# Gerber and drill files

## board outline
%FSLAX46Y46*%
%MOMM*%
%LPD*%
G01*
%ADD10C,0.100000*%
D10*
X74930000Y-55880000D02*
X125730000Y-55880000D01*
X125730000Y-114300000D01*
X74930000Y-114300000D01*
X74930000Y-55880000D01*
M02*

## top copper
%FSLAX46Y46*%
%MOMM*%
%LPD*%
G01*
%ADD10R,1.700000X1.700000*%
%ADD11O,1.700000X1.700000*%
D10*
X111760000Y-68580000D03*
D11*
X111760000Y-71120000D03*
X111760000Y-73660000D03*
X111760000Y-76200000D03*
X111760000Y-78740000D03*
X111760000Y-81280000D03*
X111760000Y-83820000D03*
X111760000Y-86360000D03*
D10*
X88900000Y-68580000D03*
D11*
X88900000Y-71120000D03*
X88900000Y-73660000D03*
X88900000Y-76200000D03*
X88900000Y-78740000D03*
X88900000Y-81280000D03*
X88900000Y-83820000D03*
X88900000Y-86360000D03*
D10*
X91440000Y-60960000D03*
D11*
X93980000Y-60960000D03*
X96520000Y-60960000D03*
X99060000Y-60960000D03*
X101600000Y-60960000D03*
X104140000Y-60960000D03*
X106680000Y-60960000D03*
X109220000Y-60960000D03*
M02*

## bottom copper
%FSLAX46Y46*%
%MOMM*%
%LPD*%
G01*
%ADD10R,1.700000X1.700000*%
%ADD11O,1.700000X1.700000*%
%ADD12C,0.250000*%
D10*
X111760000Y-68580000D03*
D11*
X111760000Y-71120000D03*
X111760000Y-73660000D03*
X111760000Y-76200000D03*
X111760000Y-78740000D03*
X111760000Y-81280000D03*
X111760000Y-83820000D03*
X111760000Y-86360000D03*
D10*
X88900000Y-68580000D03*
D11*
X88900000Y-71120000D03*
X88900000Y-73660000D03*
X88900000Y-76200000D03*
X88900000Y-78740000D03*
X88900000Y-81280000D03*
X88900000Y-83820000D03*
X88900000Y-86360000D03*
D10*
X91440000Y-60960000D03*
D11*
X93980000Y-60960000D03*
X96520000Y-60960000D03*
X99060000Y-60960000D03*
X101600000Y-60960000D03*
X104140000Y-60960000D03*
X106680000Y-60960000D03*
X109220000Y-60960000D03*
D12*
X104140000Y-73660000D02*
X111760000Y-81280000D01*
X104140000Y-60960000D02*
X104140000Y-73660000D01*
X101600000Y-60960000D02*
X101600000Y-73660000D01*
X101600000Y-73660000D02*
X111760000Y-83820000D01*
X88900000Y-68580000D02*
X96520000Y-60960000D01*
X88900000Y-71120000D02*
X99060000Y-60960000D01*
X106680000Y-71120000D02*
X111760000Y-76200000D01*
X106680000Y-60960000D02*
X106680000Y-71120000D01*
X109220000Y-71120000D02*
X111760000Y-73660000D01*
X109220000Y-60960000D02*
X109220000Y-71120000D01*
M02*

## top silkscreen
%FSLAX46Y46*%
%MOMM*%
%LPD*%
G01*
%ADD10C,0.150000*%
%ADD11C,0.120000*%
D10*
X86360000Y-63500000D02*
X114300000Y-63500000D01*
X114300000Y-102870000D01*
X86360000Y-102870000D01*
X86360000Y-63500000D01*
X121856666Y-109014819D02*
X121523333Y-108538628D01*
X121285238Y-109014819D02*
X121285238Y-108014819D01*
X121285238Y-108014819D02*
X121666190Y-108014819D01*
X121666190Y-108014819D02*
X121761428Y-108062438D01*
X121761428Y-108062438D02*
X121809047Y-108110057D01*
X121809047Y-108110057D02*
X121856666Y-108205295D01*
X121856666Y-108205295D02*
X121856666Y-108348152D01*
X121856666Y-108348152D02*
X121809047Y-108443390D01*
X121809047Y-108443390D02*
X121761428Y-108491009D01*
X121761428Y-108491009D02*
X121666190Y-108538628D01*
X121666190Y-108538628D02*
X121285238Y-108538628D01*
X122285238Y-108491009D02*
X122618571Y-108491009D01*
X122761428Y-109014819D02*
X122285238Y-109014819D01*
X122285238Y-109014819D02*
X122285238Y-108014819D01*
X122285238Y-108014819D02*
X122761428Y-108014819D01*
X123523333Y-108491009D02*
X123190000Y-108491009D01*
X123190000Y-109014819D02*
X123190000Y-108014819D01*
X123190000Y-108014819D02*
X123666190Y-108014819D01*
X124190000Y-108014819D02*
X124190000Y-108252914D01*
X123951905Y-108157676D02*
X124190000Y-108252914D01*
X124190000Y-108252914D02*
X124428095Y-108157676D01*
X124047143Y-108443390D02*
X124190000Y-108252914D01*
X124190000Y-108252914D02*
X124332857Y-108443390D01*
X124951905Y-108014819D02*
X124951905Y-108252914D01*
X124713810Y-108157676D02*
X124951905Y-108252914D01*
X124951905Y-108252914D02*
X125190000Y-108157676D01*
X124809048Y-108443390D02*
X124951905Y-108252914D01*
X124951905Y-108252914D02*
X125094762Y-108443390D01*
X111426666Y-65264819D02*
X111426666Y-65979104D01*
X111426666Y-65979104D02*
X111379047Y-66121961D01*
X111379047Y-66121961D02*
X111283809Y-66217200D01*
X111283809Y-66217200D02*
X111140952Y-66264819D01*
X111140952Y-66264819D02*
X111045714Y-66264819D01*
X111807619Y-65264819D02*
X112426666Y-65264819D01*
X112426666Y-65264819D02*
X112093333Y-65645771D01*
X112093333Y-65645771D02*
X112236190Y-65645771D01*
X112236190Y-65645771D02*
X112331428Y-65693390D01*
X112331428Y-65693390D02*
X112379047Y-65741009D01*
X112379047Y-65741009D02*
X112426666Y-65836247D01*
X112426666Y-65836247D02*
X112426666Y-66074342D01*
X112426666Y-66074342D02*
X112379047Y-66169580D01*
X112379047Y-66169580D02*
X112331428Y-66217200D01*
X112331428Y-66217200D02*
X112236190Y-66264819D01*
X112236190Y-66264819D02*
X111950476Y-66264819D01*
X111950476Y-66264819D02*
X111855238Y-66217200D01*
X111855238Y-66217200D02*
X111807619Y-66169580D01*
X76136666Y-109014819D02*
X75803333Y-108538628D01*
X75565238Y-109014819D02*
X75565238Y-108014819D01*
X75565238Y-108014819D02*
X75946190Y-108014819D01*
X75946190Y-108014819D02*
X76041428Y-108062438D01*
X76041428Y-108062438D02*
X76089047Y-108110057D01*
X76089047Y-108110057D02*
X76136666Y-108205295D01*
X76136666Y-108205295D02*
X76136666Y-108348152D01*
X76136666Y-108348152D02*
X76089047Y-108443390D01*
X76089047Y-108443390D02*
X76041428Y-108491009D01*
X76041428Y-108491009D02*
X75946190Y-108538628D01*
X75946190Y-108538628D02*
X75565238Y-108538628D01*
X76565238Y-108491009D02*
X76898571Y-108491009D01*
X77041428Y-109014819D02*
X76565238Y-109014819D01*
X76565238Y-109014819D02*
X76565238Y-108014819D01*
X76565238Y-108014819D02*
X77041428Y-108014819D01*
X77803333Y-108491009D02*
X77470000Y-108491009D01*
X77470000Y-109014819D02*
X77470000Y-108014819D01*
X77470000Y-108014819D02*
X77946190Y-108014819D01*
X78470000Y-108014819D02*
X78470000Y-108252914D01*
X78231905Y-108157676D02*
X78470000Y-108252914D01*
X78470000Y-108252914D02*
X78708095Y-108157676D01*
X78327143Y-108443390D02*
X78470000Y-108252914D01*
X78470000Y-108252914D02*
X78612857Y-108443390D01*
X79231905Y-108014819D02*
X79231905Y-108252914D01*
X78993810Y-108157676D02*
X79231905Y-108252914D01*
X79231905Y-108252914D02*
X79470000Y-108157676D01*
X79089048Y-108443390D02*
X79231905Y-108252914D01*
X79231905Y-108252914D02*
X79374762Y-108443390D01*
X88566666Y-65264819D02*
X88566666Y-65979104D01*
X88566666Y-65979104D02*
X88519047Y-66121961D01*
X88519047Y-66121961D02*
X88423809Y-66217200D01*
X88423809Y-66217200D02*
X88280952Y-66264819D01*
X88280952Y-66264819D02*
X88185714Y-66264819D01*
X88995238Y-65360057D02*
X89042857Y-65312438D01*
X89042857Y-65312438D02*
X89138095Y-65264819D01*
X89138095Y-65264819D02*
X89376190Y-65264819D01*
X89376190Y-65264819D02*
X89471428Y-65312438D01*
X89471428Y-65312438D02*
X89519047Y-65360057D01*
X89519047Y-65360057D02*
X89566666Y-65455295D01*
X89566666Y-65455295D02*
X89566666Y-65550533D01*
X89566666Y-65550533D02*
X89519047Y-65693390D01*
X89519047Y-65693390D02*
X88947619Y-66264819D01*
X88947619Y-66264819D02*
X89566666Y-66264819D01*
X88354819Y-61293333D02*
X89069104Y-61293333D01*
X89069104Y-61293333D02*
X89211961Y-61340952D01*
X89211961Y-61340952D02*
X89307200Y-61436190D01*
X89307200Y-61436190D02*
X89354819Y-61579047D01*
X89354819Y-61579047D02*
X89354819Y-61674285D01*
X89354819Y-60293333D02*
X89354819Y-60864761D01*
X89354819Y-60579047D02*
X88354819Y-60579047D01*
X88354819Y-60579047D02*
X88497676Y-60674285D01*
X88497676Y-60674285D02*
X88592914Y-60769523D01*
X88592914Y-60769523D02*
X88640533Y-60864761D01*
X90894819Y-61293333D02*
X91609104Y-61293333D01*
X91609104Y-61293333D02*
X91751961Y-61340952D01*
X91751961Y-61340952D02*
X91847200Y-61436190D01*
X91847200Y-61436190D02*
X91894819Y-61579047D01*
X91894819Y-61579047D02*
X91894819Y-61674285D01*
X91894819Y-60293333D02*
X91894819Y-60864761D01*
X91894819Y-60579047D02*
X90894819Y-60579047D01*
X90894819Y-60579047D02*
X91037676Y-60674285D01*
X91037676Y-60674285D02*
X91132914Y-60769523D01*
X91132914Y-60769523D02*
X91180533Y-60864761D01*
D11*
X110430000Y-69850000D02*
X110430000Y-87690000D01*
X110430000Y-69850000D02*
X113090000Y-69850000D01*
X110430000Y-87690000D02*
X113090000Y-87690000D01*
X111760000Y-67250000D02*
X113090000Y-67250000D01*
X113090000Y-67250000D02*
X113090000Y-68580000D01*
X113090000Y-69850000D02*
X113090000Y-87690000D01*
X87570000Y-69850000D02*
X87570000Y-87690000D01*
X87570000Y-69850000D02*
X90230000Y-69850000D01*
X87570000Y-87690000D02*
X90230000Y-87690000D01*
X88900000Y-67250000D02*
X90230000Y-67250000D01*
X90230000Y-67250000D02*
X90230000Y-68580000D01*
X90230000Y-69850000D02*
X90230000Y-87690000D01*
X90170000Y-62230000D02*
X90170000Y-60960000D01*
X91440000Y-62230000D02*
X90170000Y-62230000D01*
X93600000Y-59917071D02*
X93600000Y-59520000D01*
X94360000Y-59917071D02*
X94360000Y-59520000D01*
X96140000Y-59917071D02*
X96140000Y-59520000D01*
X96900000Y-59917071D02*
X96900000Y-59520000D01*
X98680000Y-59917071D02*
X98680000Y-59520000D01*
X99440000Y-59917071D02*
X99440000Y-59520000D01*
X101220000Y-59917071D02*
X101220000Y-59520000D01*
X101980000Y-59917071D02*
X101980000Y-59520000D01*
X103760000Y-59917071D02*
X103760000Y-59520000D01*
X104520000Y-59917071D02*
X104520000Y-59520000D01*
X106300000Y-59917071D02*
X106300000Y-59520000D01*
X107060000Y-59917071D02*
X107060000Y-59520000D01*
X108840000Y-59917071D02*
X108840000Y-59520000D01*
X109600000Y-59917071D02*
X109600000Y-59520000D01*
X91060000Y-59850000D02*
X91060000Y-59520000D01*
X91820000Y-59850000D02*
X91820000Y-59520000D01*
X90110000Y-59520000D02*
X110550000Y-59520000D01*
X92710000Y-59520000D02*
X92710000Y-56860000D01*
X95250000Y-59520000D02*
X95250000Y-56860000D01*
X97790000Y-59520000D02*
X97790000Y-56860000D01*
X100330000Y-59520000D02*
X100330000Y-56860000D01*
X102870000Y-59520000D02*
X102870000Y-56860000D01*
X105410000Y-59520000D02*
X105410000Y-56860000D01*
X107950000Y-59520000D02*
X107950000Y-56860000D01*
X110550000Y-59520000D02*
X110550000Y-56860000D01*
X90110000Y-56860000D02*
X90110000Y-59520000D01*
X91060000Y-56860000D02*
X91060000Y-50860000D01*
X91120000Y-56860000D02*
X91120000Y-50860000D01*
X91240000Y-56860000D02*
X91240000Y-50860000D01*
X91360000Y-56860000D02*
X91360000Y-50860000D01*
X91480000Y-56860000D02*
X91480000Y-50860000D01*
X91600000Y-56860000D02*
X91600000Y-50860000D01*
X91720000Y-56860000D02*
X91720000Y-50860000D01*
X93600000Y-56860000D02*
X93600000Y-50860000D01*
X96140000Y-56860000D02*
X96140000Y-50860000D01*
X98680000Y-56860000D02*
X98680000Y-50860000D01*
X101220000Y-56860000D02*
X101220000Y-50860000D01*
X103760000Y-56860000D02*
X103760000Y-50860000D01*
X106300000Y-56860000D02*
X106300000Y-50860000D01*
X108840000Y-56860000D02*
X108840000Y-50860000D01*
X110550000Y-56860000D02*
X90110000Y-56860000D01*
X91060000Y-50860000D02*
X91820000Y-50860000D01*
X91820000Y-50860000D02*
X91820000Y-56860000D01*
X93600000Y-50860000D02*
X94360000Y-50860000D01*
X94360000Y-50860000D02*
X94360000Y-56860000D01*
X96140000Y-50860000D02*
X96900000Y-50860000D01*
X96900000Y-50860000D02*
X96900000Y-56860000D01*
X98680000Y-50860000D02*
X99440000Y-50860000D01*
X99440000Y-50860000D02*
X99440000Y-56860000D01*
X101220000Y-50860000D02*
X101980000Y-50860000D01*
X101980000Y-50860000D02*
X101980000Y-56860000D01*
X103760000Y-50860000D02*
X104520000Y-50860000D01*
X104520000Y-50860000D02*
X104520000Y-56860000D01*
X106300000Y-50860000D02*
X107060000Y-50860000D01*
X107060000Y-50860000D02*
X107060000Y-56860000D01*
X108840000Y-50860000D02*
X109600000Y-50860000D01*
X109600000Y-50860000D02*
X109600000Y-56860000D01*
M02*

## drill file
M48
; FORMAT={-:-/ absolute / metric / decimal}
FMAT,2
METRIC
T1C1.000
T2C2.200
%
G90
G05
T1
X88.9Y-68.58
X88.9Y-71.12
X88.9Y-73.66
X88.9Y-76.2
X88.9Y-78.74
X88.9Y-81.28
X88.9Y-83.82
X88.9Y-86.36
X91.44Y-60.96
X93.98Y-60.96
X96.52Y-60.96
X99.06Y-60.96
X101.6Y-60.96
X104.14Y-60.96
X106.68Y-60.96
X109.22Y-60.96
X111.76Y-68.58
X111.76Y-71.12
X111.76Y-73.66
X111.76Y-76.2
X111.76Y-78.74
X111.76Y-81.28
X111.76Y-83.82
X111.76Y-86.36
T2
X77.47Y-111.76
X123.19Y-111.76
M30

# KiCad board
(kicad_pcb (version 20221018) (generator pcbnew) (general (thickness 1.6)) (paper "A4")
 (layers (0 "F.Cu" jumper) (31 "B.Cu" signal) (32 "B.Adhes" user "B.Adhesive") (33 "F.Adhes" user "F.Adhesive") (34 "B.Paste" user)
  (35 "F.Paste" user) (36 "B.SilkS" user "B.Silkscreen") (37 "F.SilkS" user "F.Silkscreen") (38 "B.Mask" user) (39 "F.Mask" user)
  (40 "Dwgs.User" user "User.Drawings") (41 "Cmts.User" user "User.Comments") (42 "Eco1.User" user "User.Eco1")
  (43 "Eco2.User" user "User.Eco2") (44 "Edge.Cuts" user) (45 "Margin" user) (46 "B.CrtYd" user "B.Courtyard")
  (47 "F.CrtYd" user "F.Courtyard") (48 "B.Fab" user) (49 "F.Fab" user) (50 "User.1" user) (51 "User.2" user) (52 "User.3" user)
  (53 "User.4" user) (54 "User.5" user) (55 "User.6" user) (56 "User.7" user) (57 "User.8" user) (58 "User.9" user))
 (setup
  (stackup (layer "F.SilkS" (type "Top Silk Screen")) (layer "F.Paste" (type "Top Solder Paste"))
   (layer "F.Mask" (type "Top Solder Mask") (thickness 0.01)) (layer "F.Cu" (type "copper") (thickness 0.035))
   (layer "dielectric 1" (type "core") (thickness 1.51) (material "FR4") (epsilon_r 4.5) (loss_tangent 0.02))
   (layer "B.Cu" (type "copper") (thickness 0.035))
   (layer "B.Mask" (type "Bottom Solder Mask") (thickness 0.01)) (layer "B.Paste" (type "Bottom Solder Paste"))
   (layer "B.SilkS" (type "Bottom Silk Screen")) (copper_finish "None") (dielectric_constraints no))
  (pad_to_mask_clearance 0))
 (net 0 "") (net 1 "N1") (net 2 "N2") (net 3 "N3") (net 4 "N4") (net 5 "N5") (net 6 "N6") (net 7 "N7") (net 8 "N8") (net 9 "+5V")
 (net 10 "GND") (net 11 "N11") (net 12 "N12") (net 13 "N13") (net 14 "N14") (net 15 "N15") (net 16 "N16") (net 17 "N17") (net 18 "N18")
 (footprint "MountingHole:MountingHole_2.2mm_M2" (layer "F.Cu") (at 123.19 111.76)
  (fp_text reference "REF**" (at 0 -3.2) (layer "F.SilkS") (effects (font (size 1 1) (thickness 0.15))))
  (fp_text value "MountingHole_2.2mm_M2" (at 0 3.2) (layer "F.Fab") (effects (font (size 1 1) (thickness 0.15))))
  (pad "" np_thru_hole circle (at 0 0) (size 2.2 2.2) (drill 2.2) (layers "F&B.Cu" "*.Mask")))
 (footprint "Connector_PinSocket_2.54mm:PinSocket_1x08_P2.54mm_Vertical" (layer "F.Cu") (at 111.76 68.58)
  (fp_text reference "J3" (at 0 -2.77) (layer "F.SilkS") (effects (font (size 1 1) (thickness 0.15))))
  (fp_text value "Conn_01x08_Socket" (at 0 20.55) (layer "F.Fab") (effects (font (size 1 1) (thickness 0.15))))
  (fp_line (start -1.33 1.27) (end -1.33 19.11) (stroke (width 0.12) (type solid)) (layer "F.SilkS"))
  (fp_line (start -1.33 1.27) (end 1.33 1.27) (stroke (width 0.12) (type solid)) (layer "F.SilkS"))
  (fp_line (start -1.33 19.11) (end 1.33 19.11) (stroke (width 0.12) (type solid)) (layer "F.SilkS"))
  (fp_line (start 0 -1.33) (end 1.33 -1.33) (stroke (width 0.12) (type solid)) (layer "F.SilkS"))
  (fp_line (start 1.33 -1.33) (end 1.33 0) (stroke (width 0.12) (type solid)) (layer "F.SilkS"))
  (fp_line (start 1.33 1.27) (end 1.33 19.11) (stroke (width 0.12) (type solid)) (layer "F.SilkS"))
  (pad "1" thru_hole rect (at 0 0) (size 1.7 1.7) (drill 1) (layers "*.Cu" "*.Mask") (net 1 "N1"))
  (pad "2" thru_hole oval (at 0 2.54) (size 1.7 1.7) (drill 1) (layers "*.Cu" "*.Mask") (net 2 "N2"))
  (pad "3" thru_hole oval (at 0 5.08) (size 1.7 1.7) (drill 1) (layers "*.Cu" "*.Mask") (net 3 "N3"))
  (pad "4" thru_hole oval (at 0 7.62) (size 1.7 1.7) (drill 1) (layers "*.Cu" "*.Mask") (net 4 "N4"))
  (pad "5" thru_hole oval (at 0 10.16) (size 1.7 1.7) (drill 1) (layers "*.Cu" "*.Mask") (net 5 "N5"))
  (pad "6" thru_hole oval (at 0 12.7) (size 1.7 1.7) (drill 1) (layers "*.Cu" "*.Mask") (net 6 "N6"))
  (pad "7" thru_hole oval (at 0 15.24) (size 1.7 1.7) (drill 1) (layers "*.Cu" "*.Mask") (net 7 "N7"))
  (pad "8" thru_hole oval (at 0 17.78) (size 1.7 1.7) (drill 1) (layers "*.Cu" "*.Mask") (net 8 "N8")))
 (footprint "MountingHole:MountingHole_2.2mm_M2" (layer "F.Cu") (at 77.47 111.76)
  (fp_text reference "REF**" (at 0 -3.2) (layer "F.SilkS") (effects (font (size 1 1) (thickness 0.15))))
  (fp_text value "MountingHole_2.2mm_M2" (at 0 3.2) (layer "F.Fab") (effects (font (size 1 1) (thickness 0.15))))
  (pad "" np_thru_hole circle (at 0 0) (size 2.2 2.2) (drill 2.2) (layers "*.Cu" "*.Mask")))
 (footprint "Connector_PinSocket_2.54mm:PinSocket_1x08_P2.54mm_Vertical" (layer "F.Cu") (at 88.9 68.58)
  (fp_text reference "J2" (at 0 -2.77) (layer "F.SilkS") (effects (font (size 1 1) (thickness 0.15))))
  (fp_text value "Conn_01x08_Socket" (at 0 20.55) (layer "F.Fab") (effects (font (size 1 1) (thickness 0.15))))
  (fp_line (start -1.33 1.27) (end -1.33 19.11) (stroke (width 0.12) (type solid)) (layer "F.SilkS"))
  (fp_line (start -1.33 1.27) (end 1.33 1.27) (stroke (width 0.12) (type solid)) (layer "F.SilkS"))
  (fp_line (start -1.33 19.11) (end 1.33 19.11) (stroke (width 0.12) (type solid)) (layer "F.SilkS"))
  (fp_line (start 0 -1.33) (end 1.33 -1.33) (stroke (width 0.12) (type solid)) (layer "F.SilkS"))
  (fp_line (start 1.33 -1.33) (end 1.33 0) (stroke (width 0.12) (type solid)) (layer "F.SilkS"))
  (fp_line (start 1.33 1.27) (end 1.33 19.11) (stroke (width 0.12) (type solid)) (layer "F.SilkS"))
  (pad "1" thru_hole rect (at 0 0) (size 1.7 1.7) (drill 1) (layers "*.Cu" "*.Mask") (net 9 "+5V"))
  (pad "2" thru_hole oval (at 0 2.54) (size 1.7 1.7) (drill 1) (layers "*.Cu" "*.Mask") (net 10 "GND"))
  (pad "3" thru_hole oval (at 0 5.08) (size 1.7 1.7) (drill 1) (layers "*.Cu" "*.Mask") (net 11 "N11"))
  (pad "4" thru_hole oval (at 0 7.62) (size 1.7 1.7) (drill 1) (layers "*.Cu" "*.Mask") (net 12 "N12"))
  (pad "5" thru_hole oval (at 0 10.16) (size 1.7 1.7) (drill 1) (layers "*.Cu" "*.Mask") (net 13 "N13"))
  (pad "6" thru_hole oval (at 0 12.7) (size 1.7 1.7) (drill 1) (layers "*.Cu" "*.Mask") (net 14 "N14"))
  (pad "7" thru_hole oval (at 0 15.24) (size 1.7 1.7) (drill 1) (layers "*.Cu" "*.Mask") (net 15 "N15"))
  (pad "8" thru_hole oval (at 0 17.78) (size 1.7 1.7) (drill 1) (layers "*.Cu" "*.Mask") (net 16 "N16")))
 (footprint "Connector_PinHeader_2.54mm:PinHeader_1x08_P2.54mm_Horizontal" (layer "F.Cu") (at 91.44 60.96 90)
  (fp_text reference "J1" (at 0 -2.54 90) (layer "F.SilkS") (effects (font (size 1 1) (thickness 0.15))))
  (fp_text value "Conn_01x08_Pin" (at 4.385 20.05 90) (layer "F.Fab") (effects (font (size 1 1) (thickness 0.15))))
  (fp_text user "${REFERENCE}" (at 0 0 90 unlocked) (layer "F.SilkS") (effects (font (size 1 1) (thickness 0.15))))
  (fp_line (start -1.27 -1.27) (end 0 -1.27) (stroke (width 0.12) (type solid)) (layer "F.SilkS"))
  (fp_line (start -1.27 0) (end -1.27 -1.27) (stroke (width 0.12) (type solid)) (layer "F.SilkS"))
  (fp_line (start 1.042929 2.16) (end 1.44 2.16) (stroke (width 0.12) (type solid)) (layer "F.SilkS"))
  (fp_line (start 1.042929 2.92) (end 1.44 2.92) (stroke (width 0.12) (type solid)) (layer "F.SilkS"))
  (fp_line (start 1.042929 4.7) (end 1.44 4.7) (stroke (width 0.12) (type solid)) (layer "F.SilkS"))
  (fp_line (start 1.042929 5.46) (end 1.44 5.46) (stroke (width 0.12) (type solid)) (layer "F.SilkS"))
  (fp_line (start 1.042929 7.24) (end 1.44 7.24) (stroke (width 0.12) (type solid)) (layer "F.SilkS"))
  (fp_line (start 1.042929 8) (end 1.44 8) (stroke (width 0.12) (type solid)) (layer "F.SilkS"))
  (fp_line (start 1.042929 9.78) (end 1.44 9.78) (stroke (width 0.12) (type solid)) (layer "F.SilkS"))
  (fp_line (start 1.042929 10.54) (end 1.44 10.54) (stroke (width 0.12) (type solid)) (layer "F.SilkS"))
  (fp_line (start 1.042929 12.32) (end 1.44 12.32) (stroke (width 0.12) (type solid)) (layer "F.SilkS"))
  (fp_line (start 1.042929 13.08) (end 1.44 13.08) (stroke (width 0.12) (type solid)) (layer "F.SilkS"))
  (fp_line (start 1.042929 14.86) (end 1.44 14.86) (stroke (width 0.12) (type solid)) (layer "F.SilkS"))
  (fp_line (start 1.042929 15.62) (end 1.44 15.62) (stroke (width 0.12) (type solid)) (layer "F.SilkS"))
  (fp_line (start 1.042929 17.4) (end 1.44 17.4) (stroke (width 0.12) (type solid)) (layer "F.SilkS"))
  (fp_line (start 1.042929 18.16) (end 1.44 18.16) (stroke (width 0.12) (type solid)) (layer "F.SilkS"))
  (fp_line (start 1.11 -0.38) (end 1.44 -0.38) (stroke (width 0.12) (type solid)) (layer "F.SilkS"))
  (fp_line (start 1.11 0.38) (end 1.44 0.38) (stroke (width 0.12) (type solid)) (layer "F.SilkS"))
  (fp_line (start 1.44 -1.33) (end 1.44 19.11) (stroke (width 0.12) (type solid)) (layer "F.SilkS"))
  (fp_line (start 1.44 1.27) (end 4.1 1.27) (stroke (width 0.12) (type solid)) (layer "F.SilkS"))
  (fp_line (start 1.44 3.81) (end 4.1 3.81) (stroke (width 0.12) (type solid)) (layer "F.SilkS"))
  (fp_line (start 1.44 6.35) (end 4.1 6.35) (stroke (width 0.12) (type solid)) (layer "F.SilkS"))
  (fp_line (start 1.44 8.89) (end 4.1 8.89) (stroke (width 0.12) (type solid)) (layer "F.SilkS"))
  (fp_line (start 1.44 11.43) (end 4.1 11.43) (stroke (width 0.12) (type solid)) (layer "F.SilkS"))
  (fp_line (start 1.44 13.97) (end 4.1 13.97) (stroke (width 0.12) (type solid)) (layer "F.SilkS"))
  (fp_line (start 1.44 16.51) (end 4.1 16.51) (stroke (width 0.12) (type solid)) (layer "F.SilkS"))
  (fp_line (start 1.44 19.11) (end 4.1 19.11) (stroke (width 0.12) (type solid)) (layer "F.SilkS"))
  (fp_line (start 4.1 -1.33) (end 1.44 -1.33) (stroke (width 0.12) (type solid)) (layer "F.SilkS"))
  (fp_line (start 4.1 -0.38) (end 10.1 -0.38) (stroke (width 0.12) (type solid)) (layer "F.SilkS"))
  (fp_line (start 4.1 -0.32) (end 10.1 -0.32) (stroke (width 0.12) (type solid)) (layer "F.SilkS"))
  (fp_line (start 4.1 -0.2) (end 10.1 -0.2) (stroke (width 0.12) (type solid)) (layer "F.SilkS"))
  (fp_line (start 4.1 -0.08) (end 10.1 -0.08) (stroke (width 0.12) (type solid)) (layer "F.SilkS"))
  (fp_line (start 4.1 0.04) (end 10.1 0.04) (stroke (width 0.12) (type solid)) (layer "F.SilkS"))
  (fp_line (start 4.1 0.16) (end 10.1 0.16) (stroke (width 0.12) (type solid)) (layer "F.SilkS"))
  (fp_line (start 4.1 0.28) (end 10.1 0.28) (stroke (width 0.12) (type solid)) (layer "F.SilkS"))
  (fp_line (start 4.1 2.16) (end 10.1 2.16) (stroke (width 0.12) (type solid)) (layer "F.SilkS"))
  (fp_line (start 4.1 4.7) (end 10.1 4.7) (stroke (width 0.12) (type solid)) (layer "F.SilkS"))
  (fp_line (start 4.1 7.24) (end 10.1 7.24) (stroke (width 0.12) (type solid)) (layer "F.SilkS"))
  (fp_line (start 4.1 9.78) (end 10.1 9.78) (stroke (width 0.12) (type solid)) (layer "F.SilkS"))
  (fp_line (start 4.1 12.32) (end 10.1 12.32) (stroke (width 0.12) (type solid)) (layer "F.SilkS"))
  (fp_line (start 4.1 14.86) (end 10.1 14.86) (stroke (width 0.12) (type solid)) (layer "F.SilkS"))
  (fp_line (start 4.1 17.4) (end 10.1 17.4) (stroke (width 0.12) (type solid)) (layer "F.SilkS"))
  (fp_line (start 4.1 19.11) (end 4.1 -1.33) (stroke (width 0.12) (type solid)) (layer "F.SilkS"))
  (fp_line (start 10.1 -0.38) (end 10.1 0.38) (stroke (width 0.12) (type solid)) (layer "F.SilkS"))
  (fp_line (start 10.1 0.38) (end 4.1 0.38) (stroke (width 0.12) (type solid)) (layer "F.SilkS"))
  (fp_line (start 10.1 2.16) (end 10.1 2.92) (stroke (width 0.12) (type solid)) (layer "F.SilkS"))
  (fp_line (start 10.1 2.92) (end 4.1 2.92) (stroke (width 0.12) (type solid)) (layer "F.SilkS"))
  (fp_line (start 10.1 4.7) (end 10.1 5.46) (stroke (width 0.12) (type solid)) (layer "F.SilkS"))
  (fp_line (start 10.1 5.46) (end 4.1 5.46) (stroke (width 0.12) (type solid)) (layer "F.SilkS"))
  (fp_line (start 10.1 7.24) (end 10.1 8) (stroke (width 0.12) (type solid)) (layer "F.SilkS"))
  (fp_line (start 10.1 8) (end 4.1 8) (stroke (width 0.12) (type solid)) (layer "F.SilkS"))
  (fp_line (start 10.1 9.78) (end 10.1 10.54) (stroke (width 0.12) (type solid)) (layer "F.SilkS"))
  (fp_line (start 10.1 10.54) (end 4.1 10.54) (stroke (width 0.12) (type solid)) (layer "F.SilkS"))
  (fp_line (start 10.1 12.32) (end 10.1 13.08) (stroke (width 0.12) (type solid)) (layer "F.SilkS"))
  (fp_line (start 10.1 13.08) (end 4.1 13.08) (stroke (width 0.12) (type solid)) (layer "F.SilkS"))
  (fp_line (start 10.1 14.86) (end 10.1 15.62) (stroke (width 0.12) (type solid)) (layer "F.SilkS"))
  (fp_line (start 10.1 15.62) (end 4.1 15.62) (stroke (width 0.12) (type solid)) (layer "F.SilkS"))
  (fp_line (start 10.1 17.4) (end 10.1 18.16) (stroke (width 0.12) (type solid)) (layer "F.SilkS"))
  (fp_line (start 10.1 18.16) (end 4.1 18.16) (stroke (width 0.12) (type solid)) (layer "F.SilkS"))
  (pad "1" thru_hole rect (at 0 0 90) (size 1.7 1.7) (drill 1) (layers "*.Cu" "*.Mask") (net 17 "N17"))
  (pad "2" thru_hole oval (at 0 2.54 90) (size 1.7 1.7) (drill 1) (layers "*.Cu" "*.Mask") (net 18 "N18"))
  (pad "3" thru_hole oval (at 0 5.08 90) (size 1.7 1.7) (drill 1) (layers "*.Cu" "*.Mask") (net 9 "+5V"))
  (pad "4" thru_hole oval (at 0 7.62 90) (size 1.7 1.7) (drill 1) (layers "*.Cu" "*.Mask") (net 10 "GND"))
  (pad "5" thru_hole oval (at 0 10.16 90) (size 1.7 1.7) (drill 1) (layers "*.Cu" "*.Mask") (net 7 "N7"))
  (pad "6" thru_hole oval (at 0 12.7 90) (size 1.7 1.7) (drill 1) (layers "*.Cu" "*.Mask") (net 6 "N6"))
  (pad "7" thru_hole oval (at 0 15.24 90) (size 1.7 1.7) (drill 1) (layers "*.Cu" "*.Mask") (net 4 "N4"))
  (pad "8" thru_hole oval (at 0 17.78 90) (size 1.7 1.7) (drill 1) (layers "*.Cu" "*.Mask") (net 3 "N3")))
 (gr_rect (start 86.36 63.5) (end 114.3 102.87) (stroke (width 0.15) (type default)) (fill none) (layer "F.SilkS"))
 (gr_rect (start 74.93 55.88) (end 125.73 114.3) (stroke (width 0.1) (type default)) (fill none) (layer "Edge.Cuts"))
 (segment (start 104.14 73.66) (end 111.76 81.28) (width 0.25) (layer "B.Cu") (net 6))
 (segment (start 104.14 60.96) (end 104.14 73.66) (width 0.25) (layer "B.Cu") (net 6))
 (segment (start 101.6 60.96) (end 101.6 73.66) (width 0.25) (layer "B.Cu") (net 7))
 (segment (start 101.6 73.66) (end 111.76 83.82) (width 0.25) (layer "B.Cu") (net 7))
 (segment (start 88.9 68.58) (end 96.52 60.96) (width 0.25) (layer "B.Cu") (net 9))
 (segment (start 88.9 71.12) (end 99.06 60.96) (width 0.25) (layer "B.Cu") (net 10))
 (segment (start 106.68 71.12) (end 111.76 76.2) (width 0.25) (layer "B.Cu") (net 4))
 (segment (start 106.68 60.96) (end 106.68 71.12) (width 0.25) (layer "B.Cu") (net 4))
 (segment (start 109.22 71.12) (end 111.76 73.66) (width 0.25) (layer "B.Cu") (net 3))
 (segment (start 109.22 60.96) (end 109.22 71.12) (width 0.25) (layer "B.Cu") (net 3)))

